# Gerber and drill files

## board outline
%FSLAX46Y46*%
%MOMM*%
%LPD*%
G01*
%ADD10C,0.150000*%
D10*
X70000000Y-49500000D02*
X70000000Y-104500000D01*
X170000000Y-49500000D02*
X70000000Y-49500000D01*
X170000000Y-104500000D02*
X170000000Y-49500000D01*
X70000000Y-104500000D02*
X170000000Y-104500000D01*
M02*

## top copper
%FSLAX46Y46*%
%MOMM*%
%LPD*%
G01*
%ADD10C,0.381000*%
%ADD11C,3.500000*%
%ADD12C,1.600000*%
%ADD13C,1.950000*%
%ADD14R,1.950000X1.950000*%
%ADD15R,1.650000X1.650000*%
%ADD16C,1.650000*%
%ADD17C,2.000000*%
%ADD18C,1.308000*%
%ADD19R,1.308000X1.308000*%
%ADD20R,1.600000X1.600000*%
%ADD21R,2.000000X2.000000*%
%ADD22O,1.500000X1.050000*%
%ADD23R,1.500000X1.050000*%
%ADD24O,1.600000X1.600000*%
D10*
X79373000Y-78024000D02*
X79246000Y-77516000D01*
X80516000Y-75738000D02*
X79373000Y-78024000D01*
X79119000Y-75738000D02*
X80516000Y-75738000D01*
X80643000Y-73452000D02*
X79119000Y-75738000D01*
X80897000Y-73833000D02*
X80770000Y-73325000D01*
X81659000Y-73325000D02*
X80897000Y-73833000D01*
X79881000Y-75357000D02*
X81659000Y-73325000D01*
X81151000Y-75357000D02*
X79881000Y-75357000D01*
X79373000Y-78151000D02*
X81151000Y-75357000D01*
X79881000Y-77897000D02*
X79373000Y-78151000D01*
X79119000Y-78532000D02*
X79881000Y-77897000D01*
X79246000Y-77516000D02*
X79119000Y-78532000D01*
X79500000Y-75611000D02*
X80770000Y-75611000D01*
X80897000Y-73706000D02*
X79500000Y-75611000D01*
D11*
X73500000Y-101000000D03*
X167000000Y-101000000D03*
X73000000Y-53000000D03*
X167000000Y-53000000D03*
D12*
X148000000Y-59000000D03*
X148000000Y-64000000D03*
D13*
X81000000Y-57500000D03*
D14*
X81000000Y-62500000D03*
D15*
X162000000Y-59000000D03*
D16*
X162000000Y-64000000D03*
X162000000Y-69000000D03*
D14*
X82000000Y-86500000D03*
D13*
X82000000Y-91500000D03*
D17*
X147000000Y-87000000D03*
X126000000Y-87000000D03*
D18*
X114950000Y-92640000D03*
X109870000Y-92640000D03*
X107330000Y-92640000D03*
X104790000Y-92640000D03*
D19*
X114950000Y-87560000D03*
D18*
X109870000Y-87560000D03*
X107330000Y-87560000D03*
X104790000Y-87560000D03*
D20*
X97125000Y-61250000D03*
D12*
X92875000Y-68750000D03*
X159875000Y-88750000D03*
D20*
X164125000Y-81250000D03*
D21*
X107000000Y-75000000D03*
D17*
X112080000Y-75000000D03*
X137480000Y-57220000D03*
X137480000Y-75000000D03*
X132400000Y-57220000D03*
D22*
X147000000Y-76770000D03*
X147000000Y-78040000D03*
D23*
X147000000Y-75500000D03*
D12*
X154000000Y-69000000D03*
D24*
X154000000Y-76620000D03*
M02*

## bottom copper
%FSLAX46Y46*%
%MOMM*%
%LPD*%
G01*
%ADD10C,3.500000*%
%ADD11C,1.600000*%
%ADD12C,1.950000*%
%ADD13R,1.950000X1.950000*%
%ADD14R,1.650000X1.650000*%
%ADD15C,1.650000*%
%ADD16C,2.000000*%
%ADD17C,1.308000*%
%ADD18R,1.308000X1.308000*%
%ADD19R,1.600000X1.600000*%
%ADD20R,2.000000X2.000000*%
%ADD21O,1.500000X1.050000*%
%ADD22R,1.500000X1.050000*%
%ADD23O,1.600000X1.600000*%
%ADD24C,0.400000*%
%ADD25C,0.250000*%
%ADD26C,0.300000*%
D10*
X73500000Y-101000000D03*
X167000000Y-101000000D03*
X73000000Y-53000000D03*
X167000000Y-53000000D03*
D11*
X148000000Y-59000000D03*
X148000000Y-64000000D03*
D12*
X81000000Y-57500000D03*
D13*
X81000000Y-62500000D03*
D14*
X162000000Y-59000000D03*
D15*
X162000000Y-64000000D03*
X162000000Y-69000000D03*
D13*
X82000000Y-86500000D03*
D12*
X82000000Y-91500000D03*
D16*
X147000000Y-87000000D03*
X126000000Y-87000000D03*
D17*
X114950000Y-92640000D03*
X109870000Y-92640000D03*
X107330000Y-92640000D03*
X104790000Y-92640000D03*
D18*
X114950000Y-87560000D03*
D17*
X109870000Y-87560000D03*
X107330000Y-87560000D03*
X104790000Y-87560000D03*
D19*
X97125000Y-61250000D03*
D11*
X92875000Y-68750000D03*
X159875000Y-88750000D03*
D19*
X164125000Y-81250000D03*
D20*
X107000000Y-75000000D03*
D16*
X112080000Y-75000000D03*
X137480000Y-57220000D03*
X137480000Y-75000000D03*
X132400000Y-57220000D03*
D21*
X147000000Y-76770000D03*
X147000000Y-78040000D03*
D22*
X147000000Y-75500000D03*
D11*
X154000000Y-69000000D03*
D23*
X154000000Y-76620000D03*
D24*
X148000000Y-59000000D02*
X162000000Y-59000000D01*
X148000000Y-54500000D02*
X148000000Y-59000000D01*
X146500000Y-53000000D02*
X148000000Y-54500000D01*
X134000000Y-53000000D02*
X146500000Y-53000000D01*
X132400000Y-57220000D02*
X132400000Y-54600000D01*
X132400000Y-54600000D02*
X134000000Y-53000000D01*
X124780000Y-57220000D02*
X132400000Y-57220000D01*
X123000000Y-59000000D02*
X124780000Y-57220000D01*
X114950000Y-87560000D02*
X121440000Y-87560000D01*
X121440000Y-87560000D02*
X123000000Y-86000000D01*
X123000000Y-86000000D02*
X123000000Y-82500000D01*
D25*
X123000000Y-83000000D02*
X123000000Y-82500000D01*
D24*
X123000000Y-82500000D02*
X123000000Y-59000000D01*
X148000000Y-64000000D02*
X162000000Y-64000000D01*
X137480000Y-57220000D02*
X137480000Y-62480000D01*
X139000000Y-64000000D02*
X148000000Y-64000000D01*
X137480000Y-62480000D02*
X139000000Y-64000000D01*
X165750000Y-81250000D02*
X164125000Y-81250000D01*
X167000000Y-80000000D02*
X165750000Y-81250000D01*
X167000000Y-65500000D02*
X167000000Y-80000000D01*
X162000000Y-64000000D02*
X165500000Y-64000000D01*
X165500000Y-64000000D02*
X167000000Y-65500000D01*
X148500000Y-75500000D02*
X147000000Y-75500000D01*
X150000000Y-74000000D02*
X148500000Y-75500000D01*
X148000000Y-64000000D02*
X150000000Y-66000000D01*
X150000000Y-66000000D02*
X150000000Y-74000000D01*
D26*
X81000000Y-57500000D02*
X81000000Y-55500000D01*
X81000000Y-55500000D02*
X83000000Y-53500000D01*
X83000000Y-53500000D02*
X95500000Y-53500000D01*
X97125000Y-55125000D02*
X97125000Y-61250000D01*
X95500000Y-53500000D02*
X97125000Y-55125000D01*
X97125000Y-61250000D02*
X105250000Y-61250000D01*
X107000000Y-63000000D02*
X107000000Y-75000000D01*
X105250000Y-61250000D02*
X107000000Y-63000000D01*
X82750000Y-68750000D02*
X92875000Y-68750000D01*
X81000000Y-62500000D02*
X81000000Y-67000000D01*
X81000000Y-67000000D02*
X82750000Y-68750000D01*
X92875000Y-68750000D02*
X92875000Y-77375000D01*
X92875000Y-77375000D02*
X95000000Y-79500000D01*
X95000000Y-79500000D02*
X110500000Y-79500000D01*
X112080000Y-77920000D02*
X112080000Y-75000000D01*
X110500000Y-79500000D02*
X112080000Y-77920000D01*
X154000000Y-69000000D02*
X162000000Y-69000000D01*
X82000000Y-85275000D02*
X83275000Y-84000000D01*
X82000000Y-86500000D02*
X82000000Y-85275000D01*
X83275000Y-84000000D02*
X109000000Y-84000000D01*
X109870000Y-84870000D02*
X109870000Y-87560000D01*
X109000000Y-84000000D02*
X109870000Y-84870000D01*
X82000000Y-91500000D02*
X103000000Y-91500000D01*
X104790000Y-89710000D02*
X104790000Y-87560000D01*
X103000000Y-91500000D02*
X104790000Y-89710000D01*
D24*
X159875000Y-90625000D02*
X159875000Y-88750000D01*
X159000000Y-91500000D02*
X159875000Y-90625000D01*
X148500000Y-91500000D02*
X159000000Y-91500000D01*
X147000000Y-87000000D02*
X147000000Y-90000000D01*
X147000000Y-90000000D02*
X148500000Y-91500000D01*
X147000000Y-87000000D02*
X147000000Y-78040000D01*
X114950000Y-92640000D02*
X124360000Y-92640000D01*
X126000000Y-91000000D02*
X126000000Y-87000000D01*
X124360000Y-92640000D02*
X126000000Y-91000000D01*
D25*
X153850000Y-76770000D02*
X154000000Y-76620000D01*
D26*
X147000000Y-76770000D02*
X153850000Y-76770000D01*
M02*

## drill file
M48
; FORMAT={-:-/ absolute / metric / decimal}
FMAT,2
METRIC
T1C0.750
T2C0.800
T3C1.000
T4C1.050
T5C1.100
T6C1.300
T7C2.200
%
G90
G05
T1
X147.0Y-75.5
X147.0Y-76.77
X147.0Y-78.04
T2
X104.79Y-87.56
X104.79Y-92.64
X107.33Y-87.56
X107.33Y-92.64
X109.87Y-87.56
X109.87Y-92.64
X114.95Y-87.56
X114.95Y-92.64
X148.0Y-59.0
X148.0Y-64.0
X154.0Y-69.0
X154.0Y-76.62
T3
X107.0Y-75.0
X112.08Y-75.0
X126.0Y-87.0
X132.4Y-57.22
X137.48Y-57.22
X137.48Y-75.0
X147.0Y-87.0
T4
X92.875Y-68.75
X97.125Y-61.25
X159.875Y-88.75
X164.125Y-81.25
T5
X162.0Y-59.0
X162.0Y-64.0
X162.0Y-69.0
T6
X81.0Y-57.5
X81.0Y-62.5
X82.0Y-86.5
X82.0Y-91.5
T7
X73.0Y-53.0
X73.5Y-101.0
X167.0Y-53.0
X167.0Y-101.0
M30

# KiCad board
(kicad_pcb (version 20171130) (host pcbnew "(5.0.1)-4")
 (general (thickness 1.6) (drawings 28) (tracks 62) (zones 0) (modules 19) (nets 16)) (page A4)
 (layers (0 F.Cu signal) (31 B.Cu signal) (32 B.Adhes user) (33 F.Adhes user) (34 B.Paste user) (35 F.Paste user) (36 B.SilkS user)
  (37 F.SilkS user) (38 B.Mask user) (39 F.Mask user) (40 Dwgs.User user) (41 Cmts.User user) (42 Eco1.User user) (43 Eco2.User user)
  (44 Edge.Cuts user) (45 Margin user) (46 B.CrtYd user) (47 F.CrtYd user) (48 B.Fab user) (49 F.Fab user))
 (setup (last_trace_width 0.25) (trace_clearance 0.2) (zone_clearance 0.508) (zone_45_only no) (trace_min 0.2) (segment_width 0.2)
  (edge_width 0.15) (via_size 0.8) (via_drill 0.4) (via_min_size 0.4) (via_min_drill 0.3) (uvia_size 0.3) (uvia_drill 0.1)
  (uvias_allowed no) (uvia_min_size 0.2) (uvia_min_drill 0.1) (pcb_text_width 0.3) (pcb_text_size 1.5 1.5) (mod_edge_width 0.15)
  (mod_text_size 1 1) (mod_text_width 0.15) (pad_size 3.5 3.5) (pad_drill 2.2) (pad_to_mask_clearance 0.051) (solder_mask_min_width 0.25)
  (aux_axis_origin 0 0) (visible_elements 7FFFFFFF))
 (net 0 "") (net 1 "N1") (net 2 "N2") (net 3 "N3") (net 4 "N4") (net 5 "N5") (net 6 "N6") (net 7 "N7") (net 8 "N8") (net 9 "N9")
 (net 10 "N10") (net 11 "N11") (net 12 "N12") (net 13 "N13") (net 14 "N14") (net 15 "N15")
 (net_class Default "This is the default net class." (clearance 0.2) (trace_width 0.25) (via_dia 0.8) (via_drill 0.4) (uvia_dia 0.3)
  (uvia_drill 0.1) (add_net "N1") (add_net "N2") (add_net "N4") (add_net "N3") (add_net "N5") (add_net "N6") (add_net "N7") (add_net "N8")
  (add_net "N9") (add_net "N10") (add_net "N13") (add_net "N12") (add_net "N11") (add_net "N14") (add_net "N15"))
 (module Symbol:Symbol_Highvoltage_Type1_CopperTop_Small (layer F.Cu) (at 79.5 76.5)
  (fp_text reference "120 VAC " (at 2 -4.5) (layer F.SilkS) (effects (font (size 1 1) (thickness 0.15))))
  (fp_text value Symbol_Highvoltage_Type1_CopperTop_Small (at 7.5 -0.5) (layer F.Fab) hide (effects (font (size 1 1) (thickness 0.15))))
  (fp_line (start -0.127 1.524) (end -0.254 1.016) (layer F.Cu) (width 0.381))
  (fp_line (start 1.016 -0.762) (end -0.127 1.524) (layer F.Cu) (width 0.381))
  (fp_line (start -0.381 -0.762) (end 1.016 -0.762) (layer F.Cu) (width 0.381))
  (fp_line (start 1.143 -3.048) (end -0.381 -0.762) (layer F.Cu) (width 0.381))
  (fp_line (start 1.397 -2.667) (end 1.27 -3.175) (layer F.Cu) (width 0.381))
  (fp_line (start 2.159 -3.175) (end 1.397 -2.667) (layer F.Cu) (width 0.381))
  (fp_line (start 0.381 -1.143) (end 2.159 -3.175) (layer F.Cu) (width 0.381))
  (fp_line (start 1.651 -1.143) (end 0.381 -1.143) (layer F.Cu) (width 0.381))
  (fp_line (start -0.127 1.651) (end 1.651 -1.143) (layer F.Cu) (width 0.381))
  (fp_line (start 0.381 1.397) (end -0.127 1.651) (layer F.Cu) (width 0.381))
  (fp_line (start -0.381 2.032) (end 0.381 1.397) (layer F.Cu) (width 0.381))
  (fp_line (start -0.254 1.016) (end -0.381 2.032) (layer F.Cu) (width 0.381))
  (fp_line (start 0 -0.889) (end 1.27 -0.889) (layer F.Cu) (width 0.381))
  (fp_line (start 1.397 -2.794) (end 0 -0.889) (layer F.Cu) (width 0.381)))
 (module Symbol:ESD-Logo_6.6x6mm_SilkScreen (layer F.Cu) (at 147 68)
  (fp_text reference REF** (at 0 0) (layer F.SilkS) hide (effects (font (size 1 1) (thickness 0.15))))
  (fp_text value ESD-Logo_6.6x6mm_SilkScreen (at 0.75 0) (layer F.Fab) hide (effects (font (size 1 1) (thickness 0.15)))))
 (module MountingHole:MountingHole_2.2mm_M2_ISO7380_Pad (layer F.Cu) (at 73.5 101)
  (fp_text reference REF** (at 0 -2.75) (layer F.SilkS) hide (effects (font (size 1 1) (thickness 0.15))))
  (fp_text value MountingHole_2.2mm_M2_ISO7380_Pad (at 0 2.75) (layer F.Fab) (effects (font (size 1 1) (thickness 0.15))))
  (pad 1 thru_hole circle (at 0 0) (size 3.5 3.5) (drill 2.2) (layers *.Cu *.Mask)))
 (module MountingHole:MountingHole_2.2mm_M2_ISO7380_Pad (layer F.Cu) (at 167 101)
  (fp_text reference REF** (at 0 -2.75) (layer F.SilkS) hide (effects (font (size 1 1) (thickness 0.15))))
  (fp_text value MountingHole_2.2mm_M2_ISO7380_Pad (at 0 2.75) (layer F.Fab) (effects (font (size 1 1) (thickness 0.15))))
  (pad 1 thru_hole circle (at 0 0) (size 3.5 3.5) (drill 2.2) (layers *.Cu *.Mask)))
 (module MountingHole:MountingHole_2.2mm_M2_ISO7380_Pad (layer F.Cu) (at 73 53)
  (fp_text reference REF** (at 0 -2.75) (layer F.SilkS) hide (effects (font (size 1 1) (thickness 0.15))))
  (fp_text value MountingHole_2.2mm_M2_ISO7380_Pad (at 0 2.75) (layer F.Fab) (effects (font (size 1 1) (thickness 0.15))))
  (pad 1 thru_hole circle (at 0 0) (size 3.5 3.5) (drill 2.2) (layers *.Cu *.Mask)))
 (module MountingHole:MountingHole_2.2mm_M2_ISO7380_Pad (layer F.Cu) (at 167 53)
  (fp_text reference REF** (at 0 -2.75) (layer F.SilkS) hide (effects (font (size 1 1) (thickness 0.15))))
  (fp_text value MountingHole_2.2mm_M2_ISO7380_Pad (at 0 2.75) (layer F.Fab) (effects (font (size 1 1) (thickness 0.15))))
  (pad 1 thru_hole circle (at 0 0) (size 3.5 3.5) (drill 2.2) (layers *.Cu *.Mask)))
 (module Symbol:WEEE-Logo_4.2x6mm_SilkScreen (layer F.Cu) (at 152.5 99.5)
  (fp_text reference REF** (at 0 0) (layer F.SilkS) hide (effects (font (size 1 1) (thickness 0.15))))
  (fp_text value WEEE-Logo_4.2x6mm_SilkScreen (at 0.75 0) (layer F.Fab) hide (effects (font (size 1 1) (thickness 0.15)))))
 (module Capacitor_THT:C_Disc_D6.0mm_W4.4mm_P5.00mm (layer F.Cu) (at 148 59 270)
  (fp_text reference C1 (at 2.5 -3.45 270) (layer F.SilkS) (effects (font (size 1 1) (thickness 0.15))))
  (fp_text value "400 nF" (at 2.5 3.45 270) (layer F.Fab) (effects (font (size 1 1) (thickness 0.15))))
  (pad 1 thru_hole circle (at 0 0 270) (size 1.6 1.6) (drill 0.8) (layers *.Cu *.Mask) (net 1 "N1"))
  (pad 2 thru_hole circle (at 5 0 270) (size 1.6 1.6) (drill 0.8) (layers *.Cu *.Mask) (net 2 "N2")))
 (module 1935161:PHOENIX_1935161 (layer F.Cu) (at 81 60 90)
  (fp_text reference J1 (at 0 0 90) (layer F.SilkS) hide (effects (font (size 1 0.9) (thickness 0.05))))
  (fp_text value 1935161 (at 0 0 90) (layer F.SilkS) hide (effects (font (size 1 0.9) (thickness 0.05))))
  (pad 2 thru_hole circle (at 2.5 0 90) (size 1.95 1.95) (drill 1.3) (layers *.Cu *.Mask) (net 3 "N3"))
  (pad 1 thru_hole rect (at -2.5 0 90) (size 1.95 1.95) (drill 1.3) (layers *.Cu *.Mask) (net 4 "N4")))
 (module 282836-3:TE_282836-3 (layer F.Cu) (at 162 64 270)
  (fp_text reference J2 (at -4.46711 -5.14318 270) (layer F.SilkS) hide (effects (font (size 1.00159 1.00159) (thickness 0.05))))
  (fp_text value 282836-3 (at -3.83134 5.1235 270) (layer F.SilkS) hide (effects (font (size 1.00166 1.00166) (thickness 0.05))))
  (pad 1 thru_hole rect (at -5 0 270) (size 1.65 1.65) (drill 1.1) (layers *.Cu *.Mask) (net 1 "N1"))
  (pad 2 thru_hole circle (at 0 0 270) (size 1.65 1.65) (drill 1.1) (layers *.Cu *.Mask) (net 2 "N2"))
  (pad 3 thru_hole circle (at 5 0 270) (size 1.65 1.65) (drill 1.1) (layers *.Cu *.Mask) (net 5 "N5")))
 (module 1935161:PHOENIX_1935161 (layer F.Cu) (at 82 89 270)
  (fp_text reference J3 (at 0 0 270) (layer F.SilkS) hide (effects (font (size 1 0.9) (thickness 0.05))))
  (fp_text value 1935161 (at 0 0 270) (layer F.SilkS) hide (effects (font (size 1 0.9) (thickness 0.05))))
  (pad 1 thru_hole rect (at -2.5 0 270) (size 1.95 1.95) (drill 1.3) (layers *.Cu *.Mask) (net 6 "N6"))
  (pad 2 thru_hole circle (at 2.5 0 270) (size 1.95 1.95) (drill 1.3) (layers *.Cu *.Mask) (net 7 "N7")))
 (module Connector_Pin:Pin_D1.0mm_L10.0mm (layer F.Cu) (at 147 87)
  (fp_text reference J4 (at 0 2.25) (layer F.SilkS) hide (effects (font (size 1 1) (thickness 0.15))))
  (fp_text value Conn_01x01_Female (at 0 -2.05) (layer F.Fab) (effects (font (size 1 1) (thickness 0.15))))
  (pad 1 thru_hole circle (at 0 0) (size 2 2) (drill 1) (layers *.Cu *.Mask) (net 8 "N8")))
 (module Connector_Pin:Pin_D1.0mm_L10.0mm (layer F.Cu) (at 126 87)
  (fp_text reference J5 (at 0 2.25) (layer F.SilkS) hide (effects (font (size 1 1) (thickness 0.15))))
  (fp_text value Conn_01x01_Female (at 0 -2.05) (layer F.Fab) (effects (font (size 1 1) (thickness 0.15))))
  (pad 1 thru_hole circle (at 0 0) (size 2 2) (drill 1) (layers *.Cu *.Mask) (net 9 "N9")))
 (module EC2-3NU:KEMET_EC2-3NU (layer F.Cu) (at 108.5 90 270)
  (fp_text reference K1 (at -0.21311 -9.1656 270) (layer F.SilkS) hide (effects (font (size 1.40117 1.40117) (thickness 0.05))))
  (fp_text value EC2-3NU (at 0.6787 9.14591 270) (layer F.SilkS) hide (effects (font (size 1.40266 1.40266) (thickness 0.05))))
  (pad 12 thru_hole circle (at 2.64 -6.45 180) (size 1.308 1.308) (drill 0.8) (layers *.Cu *.Mask) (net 9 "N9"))
  (pad 10 thru_hole circle (at 2.64 -1.37 180) (size 1.308 1.308) (drill 0.8) (layers *.Cu *.Mask) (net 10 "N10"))
  (pad 9 thru_hole circle (at 2.64 1.17 180) (size 1.308 1.308) (drill 0.8) (layers *.Cu *.Mask) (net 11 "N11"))
  (pad 8 thru_hole circle (at 2.64 3.71 180) (size 1.308 1.308) (drill 0.8) (layers *.Cu *.Mask) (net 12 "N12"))
  (pad 1 thru_hole rect (at -2.44 -6.45 180) (size 1.308 1.308) (drill 0.8) (layers *.Cu *.Mask) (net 1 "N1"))
  (pad 3 thru_hole circle (at -2.44 -1.37 180) (size 1.308 1.308) (drill 0.8) (layers *.Cu *.Mask) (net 6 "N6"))
  (pad 4 thru_hole circle (at -2.44 1.17 180) (size 1.308 1.308) (drill 0.8) (layers *.Cu *.Mask) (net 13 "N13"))
  (pad 5 thru_hole circle (at -2.44 3.71 180) (size 1.308 1.308) (drill 0.8) (layers *.Cu *.Mask) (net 7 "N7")))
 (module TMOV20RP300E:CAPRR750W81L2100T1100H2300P (layer F.Cu) (at 95 65 270)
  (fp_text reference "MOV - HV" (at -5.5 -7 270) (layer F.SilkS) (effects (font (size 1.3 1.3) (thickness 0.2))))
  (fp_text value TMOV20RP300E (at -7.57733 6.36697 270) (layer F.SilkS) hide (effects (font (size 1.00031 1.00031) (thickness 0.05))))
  (pad 1 thru_hole rect (at -3.75 -2.125 270) (size 1.6 1.6) (drill 1.05) (layers *.Cu *.Mask) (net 3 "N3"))
  (pad 2 thru_hole circle (at 3.75 2.125 270) (size 1.6 1.6) (drill 1.05) (layers *.Cu *.Mask) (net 4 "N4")))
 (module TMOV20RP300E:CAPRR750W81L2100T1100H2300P (layer F.Cu) (at 162 85 270)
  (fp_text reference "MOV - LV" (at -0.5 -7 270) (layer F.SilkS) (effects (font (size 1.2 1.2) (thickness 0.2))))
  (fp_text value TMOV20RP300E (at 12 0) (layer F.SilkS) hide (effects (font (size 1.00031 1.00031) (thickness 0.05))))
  (pad 2 thru_hole circle (at 3.75 2.125 270) (size 1.6 1.6) (drill 1.05) (layers *.Cu *.Mask) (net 8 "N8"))
  (pad 1 thru_hole rect (at -3.75 -2.125 270) (size 1.6 1.6) (drill 1.05) (layers *.Cu *.Mask) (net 2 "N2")))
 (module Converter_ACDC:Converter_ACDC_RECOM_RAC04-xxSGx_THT (layer F.Cu) (at 107 75 90)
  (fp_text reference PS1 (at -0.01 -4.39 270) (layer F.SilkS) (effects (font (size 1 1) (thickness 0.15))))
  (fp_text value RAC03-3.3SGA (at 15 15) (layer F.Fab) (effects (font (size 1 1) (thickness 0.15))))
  (pad 1 thru_hole rect (at 0 0 180) (size 2 2) (drill 1) (layers *.Cu *.Mask) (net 3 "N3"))
  (pad 2 thru_hole circle (at 0 5.08 180) (size 2 2) (drill 1) (layers *.Cu *.Mask) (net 4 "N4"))
  (pad 4 thru_hole circle (at 17.78 30.48 180) (size 2 2) (drill 1) (layers *.Cu *.Mask) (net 2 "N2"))
  (pad 3 thru_hole circle (at 0 30.48 270) (size 2 2) (drill 1) (layers *.Cu *.Mask) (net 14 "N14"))
  (pad 5 thru_hole circle (at 17.78 25.4 180) (size 2 2) (drill 1) (layers *.Cu *.Mask) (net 1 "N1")))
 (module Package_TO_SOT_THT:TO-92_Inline (layer F.Cu) (at 147 75.5 270)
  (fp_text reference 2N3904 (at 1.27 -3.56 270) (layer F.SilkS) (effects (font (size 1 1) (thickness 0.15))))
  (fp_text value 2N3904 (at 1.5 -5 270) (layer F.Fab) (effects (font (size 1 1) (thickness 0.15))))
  (pad 2 thru_hole oval (at 1.27 0 270) (size 1.05 1.5) (drill 0.75) (layers *.Cu *.Mask) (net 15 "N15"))
  (pad 3 thru_hole oval (at 2.54 0 270) (size 1.05 1.5) (drill 0.75) (layers *.Cu *.Mask) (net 8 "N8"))
  (pad 1 thru_hole rect (at 0 0 270) (size 1.05 1.5) (drill 0.75) (layers *.Cu *.Mask) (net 2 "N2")))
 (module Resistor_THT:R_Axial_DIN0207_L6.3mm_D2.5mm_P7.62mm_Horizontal (layer F.Cu) (at 154 69 270)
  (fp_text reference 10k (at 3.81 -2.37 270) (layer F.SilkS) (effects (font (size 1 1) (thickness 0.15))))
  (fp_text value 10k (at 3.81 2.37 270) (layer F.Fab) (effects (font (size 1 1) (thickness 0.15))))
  (pad 1 thru_hole circle (at 0 0 270) (size 1.6 1.6) (drill 0.8) (layers *.Cu *.Mask) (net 5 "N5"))
  (pad 2 thru_hole oval (at 7.62 0 270) (size 1.6 1.6) (drill 0.8) (layers *.Cu *.Mask) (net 15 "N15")))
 (gr_line (start 70 49.5) (end 70 104.5) (layer Edge.Cuts) (width 0.15))
 (gr_line (start 170 49.5) (end 70 49.5) (layer Edge.Cuts) (width 0.15))
 (gr_line (start 170 104.5) (end 170 49.5) (layer Edge.Cuts) (width 0.15))
 (gr_line (start 70 104.5) (end 170 104.5) (layer Edge.Cuts) (width 0.15))
 (segment (start 148 59) (end 162 59) (width 0.4) (layer B.Cu) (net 1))
 (segment (start 148 54.5) (end 148 59) (width 0.4) (layer B.Cu) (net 1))
 (segment (start 146.5 53) (end 148 54.5) (width 0.4) (layer B.Cu) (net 1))
 (segment (start 134 53) (end 146.5 53) (width 0.4) (layer B.Cu) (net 1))
 (segment (start 132.4 57.22) (end 132.4 54.6) (width 0.4) (layer B.Cu) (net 1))
 (segment (start 132.4 54.6) (end 134 53) (width 0.4) (layer B.Cu) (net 1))
 (segment (start 124.78 57.22) (end 132.4 57.22) (width 0.4) (layer B.Cu) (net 1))
 (segment (start 123 59) (end 124.78 57.22) (width 0.4) (layer B.Cu) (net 1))
 (segment (start 114.95 87.56) (end 121.44 87.56) (width 0.4) (layer B.Cu) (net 1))
 (segment (start 121.44 87.56) (end 123 86) (width 0.4) (layer B.Cu) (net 1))
 (segment (start 123 86) (end 123 82.5) (width 0.4) (layer B.Cu) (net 1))
 (segment (start 123 83) (end 123 82.5) (width 0.25) (layer B.Cu) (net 1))
 (segment (start 123 82.5) (end 123 59) (width 0.4) (layer B.Cu) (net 1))
 (segment (start 148 64) (end 162 64) (width 0.4) (layer B.Cu) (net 2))
 (segment (start 137.48 57.22) (end 137.48 62.48) (width 0.4) (layer B.Cu) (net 2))
 (segment (start 139 64) (end 148 64) (width 0.4) (layer B.Cu) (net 2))
 (segment (start 137.48 62.48) (end 139 64) (width 0.4) (layer B.Cu) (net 2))
 (segment (start 165.75 81.25) (end 164.125 81.25) (width 0.4) (layer B.Cu) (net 2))
 (segment (start 167 80) (end 165.75 81.25) (width 0.4) (layer B.Cu) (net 2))
 (segment (start 167 65.5) (end 167 80) (width 0.4) (layer B.Cu) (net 2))
 (segment (start 162 64) (end 165.5 64) (width 0.4) (layer B.Cu) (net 2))
 (segment (start 165.5 64) (end 167 65.5) (width 0.4) (layer B.Cu) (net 2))
 (segment (start 148.5 75.5) (end 147 75.5) (width 0.4) (layer B.Cu) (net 2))
 (segment (start 150 74) (end 148.5 75.5) (width 0.4) (layer B.Cu) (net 2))
 (segment (start 148 64) (end 150 66) (width 0.4) (layer B.Cu) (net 2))
 (segment (start 150 66) (end 150 74) (width 0.4) (layer B.Cu) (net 2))
 (segment (start 81 57.5) (end 81 55.5) (width 0.3) (layer B.Cu) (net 3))
 (segment (start 81 55.5) (end 83 53.5) (width 0.3) (layer B.Cu) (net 3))
 (segment (start 83 53.5) (end 95.5 53.5) (width 0.3) (layer B.Cu) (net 3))
 (segment (start 97.125 55.125) (end 97.125 61.25) (width 0.3) (layer B.Cu) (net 3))
 (segment (start 95.5 53.5) (end 97.125 55.125) (width 0.3) (layer B.Cu) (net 3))
 (segment (start 97.125 61.25) (end 105.25 61.25) (width 0.3) (layer B.Cu) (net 3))
 (segment (start 107 63) (end 107 75) (width 0.3) (layer B.Cu) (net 3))
 (segment (start 105.25 61.25) (end 107 63) (width 0.3) (layer B.Cu) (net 3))
 (segment (start 82.75 68.75) (end 92.875 68.75) (width 0.3) (layer B.Cu) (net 4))
 (segment (start 81 62.5) (end 81 67) (width 0.3) (layer B.Cu) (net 4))
 (segment (start 81 67) (end 82.75 68.75) (width 0.3) (layer B.Cu) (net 4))
 (segment (start 92.875 68.75) (end 92.875 77.375) (width 0.3) (layer B.Cu) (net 4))
 (segment (start 92.875 77.375) (end 95 79.5) (width 0.3) (layer B.Cu) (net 4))
 (segment (start 95 79.5) (end 110.5 79.5) (width 0.3) (layer B.Cu) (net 4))
 (segment (start 112.08 77.92) (end 112.08 75) (width 0.3) (layer B.Cu) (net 4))
 (segment (start 110.5 79.5) (end 112.08 77.92) (width 0.3) (layer B.Cu) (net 4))
 (segment (start 154 69) (end 162 69) (width 0.3) (layer B.Cu) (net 5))
 (segment (start 82 85.275) (end 83.275 84) (width 0.3) (layer B.Cu) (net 6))
 (segment (start 82 86.5) (end 82 85.275) (width 0.3) (layer B.Cu) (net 6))
 (segment (start 83.275 84) (end 109 84) (width 0.3) (layer B.Cu) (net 6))
 (segment (start 109.87 84.87) (end 109.87 87.56) (width 0.3) (layer B.Cu) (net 6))
 (segment (start 109 84) (end 109.87 84.87) (width 0.3) (layer B.Cu) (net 6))
 (segment (start 82 91.5) (end 103 91.5) (width 0.3) (layer B.Cu) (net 7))
 (segment (start 104.79 89.71) (end 104.79 87.56) (width 0.3) (layer B.Cu) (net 7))
 (segment (start 103 91.5) (end 104.79 89.71) (width 0.3) (layer B.Cu) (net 7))
 (segment (start 159.875 90.625) (end 159.875 88.75) (width 0.4) (layer B.Cu) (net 8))
 (segment (start 159 91.5) (end 159.875 90.625) (width 0.4) (layer B.Cu) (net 8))
 (segment (start 148.5 91.5) (end 159 91.5) (width 0.4) (layer B.Cu) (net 8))
 (segment (start 147 87) (end 147 90) (width 0.4) (layer B.Cu) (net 8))
 (segment (start 147 90) (end 148.5 91.5) (width 0.4) (layer B.Cu) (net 8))
 (segment (start 147 87) (end 147 78.04) (width 0.4) (layer B.Cu) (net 8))
 (segment (start 114.95 92.64) (end 124.36 92.64) (width 0.4) (layer B.Cu) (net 9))
 (segment (start 126 91) (end 126 87) (width 0.4) (layer B.Cu) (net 9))
 (segment (start 124.36 92.64) (end 126 91) (width 0.4) (layer B.Cu) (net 9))
 (segment (start 153.85 76.77) (end 154 76.62) (width 0.25) (layer B.Cu) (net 15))
 (segment (start 147 76.77) (end 153.85 76.77) (width 0.3) (layer B.Cu) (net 15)))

